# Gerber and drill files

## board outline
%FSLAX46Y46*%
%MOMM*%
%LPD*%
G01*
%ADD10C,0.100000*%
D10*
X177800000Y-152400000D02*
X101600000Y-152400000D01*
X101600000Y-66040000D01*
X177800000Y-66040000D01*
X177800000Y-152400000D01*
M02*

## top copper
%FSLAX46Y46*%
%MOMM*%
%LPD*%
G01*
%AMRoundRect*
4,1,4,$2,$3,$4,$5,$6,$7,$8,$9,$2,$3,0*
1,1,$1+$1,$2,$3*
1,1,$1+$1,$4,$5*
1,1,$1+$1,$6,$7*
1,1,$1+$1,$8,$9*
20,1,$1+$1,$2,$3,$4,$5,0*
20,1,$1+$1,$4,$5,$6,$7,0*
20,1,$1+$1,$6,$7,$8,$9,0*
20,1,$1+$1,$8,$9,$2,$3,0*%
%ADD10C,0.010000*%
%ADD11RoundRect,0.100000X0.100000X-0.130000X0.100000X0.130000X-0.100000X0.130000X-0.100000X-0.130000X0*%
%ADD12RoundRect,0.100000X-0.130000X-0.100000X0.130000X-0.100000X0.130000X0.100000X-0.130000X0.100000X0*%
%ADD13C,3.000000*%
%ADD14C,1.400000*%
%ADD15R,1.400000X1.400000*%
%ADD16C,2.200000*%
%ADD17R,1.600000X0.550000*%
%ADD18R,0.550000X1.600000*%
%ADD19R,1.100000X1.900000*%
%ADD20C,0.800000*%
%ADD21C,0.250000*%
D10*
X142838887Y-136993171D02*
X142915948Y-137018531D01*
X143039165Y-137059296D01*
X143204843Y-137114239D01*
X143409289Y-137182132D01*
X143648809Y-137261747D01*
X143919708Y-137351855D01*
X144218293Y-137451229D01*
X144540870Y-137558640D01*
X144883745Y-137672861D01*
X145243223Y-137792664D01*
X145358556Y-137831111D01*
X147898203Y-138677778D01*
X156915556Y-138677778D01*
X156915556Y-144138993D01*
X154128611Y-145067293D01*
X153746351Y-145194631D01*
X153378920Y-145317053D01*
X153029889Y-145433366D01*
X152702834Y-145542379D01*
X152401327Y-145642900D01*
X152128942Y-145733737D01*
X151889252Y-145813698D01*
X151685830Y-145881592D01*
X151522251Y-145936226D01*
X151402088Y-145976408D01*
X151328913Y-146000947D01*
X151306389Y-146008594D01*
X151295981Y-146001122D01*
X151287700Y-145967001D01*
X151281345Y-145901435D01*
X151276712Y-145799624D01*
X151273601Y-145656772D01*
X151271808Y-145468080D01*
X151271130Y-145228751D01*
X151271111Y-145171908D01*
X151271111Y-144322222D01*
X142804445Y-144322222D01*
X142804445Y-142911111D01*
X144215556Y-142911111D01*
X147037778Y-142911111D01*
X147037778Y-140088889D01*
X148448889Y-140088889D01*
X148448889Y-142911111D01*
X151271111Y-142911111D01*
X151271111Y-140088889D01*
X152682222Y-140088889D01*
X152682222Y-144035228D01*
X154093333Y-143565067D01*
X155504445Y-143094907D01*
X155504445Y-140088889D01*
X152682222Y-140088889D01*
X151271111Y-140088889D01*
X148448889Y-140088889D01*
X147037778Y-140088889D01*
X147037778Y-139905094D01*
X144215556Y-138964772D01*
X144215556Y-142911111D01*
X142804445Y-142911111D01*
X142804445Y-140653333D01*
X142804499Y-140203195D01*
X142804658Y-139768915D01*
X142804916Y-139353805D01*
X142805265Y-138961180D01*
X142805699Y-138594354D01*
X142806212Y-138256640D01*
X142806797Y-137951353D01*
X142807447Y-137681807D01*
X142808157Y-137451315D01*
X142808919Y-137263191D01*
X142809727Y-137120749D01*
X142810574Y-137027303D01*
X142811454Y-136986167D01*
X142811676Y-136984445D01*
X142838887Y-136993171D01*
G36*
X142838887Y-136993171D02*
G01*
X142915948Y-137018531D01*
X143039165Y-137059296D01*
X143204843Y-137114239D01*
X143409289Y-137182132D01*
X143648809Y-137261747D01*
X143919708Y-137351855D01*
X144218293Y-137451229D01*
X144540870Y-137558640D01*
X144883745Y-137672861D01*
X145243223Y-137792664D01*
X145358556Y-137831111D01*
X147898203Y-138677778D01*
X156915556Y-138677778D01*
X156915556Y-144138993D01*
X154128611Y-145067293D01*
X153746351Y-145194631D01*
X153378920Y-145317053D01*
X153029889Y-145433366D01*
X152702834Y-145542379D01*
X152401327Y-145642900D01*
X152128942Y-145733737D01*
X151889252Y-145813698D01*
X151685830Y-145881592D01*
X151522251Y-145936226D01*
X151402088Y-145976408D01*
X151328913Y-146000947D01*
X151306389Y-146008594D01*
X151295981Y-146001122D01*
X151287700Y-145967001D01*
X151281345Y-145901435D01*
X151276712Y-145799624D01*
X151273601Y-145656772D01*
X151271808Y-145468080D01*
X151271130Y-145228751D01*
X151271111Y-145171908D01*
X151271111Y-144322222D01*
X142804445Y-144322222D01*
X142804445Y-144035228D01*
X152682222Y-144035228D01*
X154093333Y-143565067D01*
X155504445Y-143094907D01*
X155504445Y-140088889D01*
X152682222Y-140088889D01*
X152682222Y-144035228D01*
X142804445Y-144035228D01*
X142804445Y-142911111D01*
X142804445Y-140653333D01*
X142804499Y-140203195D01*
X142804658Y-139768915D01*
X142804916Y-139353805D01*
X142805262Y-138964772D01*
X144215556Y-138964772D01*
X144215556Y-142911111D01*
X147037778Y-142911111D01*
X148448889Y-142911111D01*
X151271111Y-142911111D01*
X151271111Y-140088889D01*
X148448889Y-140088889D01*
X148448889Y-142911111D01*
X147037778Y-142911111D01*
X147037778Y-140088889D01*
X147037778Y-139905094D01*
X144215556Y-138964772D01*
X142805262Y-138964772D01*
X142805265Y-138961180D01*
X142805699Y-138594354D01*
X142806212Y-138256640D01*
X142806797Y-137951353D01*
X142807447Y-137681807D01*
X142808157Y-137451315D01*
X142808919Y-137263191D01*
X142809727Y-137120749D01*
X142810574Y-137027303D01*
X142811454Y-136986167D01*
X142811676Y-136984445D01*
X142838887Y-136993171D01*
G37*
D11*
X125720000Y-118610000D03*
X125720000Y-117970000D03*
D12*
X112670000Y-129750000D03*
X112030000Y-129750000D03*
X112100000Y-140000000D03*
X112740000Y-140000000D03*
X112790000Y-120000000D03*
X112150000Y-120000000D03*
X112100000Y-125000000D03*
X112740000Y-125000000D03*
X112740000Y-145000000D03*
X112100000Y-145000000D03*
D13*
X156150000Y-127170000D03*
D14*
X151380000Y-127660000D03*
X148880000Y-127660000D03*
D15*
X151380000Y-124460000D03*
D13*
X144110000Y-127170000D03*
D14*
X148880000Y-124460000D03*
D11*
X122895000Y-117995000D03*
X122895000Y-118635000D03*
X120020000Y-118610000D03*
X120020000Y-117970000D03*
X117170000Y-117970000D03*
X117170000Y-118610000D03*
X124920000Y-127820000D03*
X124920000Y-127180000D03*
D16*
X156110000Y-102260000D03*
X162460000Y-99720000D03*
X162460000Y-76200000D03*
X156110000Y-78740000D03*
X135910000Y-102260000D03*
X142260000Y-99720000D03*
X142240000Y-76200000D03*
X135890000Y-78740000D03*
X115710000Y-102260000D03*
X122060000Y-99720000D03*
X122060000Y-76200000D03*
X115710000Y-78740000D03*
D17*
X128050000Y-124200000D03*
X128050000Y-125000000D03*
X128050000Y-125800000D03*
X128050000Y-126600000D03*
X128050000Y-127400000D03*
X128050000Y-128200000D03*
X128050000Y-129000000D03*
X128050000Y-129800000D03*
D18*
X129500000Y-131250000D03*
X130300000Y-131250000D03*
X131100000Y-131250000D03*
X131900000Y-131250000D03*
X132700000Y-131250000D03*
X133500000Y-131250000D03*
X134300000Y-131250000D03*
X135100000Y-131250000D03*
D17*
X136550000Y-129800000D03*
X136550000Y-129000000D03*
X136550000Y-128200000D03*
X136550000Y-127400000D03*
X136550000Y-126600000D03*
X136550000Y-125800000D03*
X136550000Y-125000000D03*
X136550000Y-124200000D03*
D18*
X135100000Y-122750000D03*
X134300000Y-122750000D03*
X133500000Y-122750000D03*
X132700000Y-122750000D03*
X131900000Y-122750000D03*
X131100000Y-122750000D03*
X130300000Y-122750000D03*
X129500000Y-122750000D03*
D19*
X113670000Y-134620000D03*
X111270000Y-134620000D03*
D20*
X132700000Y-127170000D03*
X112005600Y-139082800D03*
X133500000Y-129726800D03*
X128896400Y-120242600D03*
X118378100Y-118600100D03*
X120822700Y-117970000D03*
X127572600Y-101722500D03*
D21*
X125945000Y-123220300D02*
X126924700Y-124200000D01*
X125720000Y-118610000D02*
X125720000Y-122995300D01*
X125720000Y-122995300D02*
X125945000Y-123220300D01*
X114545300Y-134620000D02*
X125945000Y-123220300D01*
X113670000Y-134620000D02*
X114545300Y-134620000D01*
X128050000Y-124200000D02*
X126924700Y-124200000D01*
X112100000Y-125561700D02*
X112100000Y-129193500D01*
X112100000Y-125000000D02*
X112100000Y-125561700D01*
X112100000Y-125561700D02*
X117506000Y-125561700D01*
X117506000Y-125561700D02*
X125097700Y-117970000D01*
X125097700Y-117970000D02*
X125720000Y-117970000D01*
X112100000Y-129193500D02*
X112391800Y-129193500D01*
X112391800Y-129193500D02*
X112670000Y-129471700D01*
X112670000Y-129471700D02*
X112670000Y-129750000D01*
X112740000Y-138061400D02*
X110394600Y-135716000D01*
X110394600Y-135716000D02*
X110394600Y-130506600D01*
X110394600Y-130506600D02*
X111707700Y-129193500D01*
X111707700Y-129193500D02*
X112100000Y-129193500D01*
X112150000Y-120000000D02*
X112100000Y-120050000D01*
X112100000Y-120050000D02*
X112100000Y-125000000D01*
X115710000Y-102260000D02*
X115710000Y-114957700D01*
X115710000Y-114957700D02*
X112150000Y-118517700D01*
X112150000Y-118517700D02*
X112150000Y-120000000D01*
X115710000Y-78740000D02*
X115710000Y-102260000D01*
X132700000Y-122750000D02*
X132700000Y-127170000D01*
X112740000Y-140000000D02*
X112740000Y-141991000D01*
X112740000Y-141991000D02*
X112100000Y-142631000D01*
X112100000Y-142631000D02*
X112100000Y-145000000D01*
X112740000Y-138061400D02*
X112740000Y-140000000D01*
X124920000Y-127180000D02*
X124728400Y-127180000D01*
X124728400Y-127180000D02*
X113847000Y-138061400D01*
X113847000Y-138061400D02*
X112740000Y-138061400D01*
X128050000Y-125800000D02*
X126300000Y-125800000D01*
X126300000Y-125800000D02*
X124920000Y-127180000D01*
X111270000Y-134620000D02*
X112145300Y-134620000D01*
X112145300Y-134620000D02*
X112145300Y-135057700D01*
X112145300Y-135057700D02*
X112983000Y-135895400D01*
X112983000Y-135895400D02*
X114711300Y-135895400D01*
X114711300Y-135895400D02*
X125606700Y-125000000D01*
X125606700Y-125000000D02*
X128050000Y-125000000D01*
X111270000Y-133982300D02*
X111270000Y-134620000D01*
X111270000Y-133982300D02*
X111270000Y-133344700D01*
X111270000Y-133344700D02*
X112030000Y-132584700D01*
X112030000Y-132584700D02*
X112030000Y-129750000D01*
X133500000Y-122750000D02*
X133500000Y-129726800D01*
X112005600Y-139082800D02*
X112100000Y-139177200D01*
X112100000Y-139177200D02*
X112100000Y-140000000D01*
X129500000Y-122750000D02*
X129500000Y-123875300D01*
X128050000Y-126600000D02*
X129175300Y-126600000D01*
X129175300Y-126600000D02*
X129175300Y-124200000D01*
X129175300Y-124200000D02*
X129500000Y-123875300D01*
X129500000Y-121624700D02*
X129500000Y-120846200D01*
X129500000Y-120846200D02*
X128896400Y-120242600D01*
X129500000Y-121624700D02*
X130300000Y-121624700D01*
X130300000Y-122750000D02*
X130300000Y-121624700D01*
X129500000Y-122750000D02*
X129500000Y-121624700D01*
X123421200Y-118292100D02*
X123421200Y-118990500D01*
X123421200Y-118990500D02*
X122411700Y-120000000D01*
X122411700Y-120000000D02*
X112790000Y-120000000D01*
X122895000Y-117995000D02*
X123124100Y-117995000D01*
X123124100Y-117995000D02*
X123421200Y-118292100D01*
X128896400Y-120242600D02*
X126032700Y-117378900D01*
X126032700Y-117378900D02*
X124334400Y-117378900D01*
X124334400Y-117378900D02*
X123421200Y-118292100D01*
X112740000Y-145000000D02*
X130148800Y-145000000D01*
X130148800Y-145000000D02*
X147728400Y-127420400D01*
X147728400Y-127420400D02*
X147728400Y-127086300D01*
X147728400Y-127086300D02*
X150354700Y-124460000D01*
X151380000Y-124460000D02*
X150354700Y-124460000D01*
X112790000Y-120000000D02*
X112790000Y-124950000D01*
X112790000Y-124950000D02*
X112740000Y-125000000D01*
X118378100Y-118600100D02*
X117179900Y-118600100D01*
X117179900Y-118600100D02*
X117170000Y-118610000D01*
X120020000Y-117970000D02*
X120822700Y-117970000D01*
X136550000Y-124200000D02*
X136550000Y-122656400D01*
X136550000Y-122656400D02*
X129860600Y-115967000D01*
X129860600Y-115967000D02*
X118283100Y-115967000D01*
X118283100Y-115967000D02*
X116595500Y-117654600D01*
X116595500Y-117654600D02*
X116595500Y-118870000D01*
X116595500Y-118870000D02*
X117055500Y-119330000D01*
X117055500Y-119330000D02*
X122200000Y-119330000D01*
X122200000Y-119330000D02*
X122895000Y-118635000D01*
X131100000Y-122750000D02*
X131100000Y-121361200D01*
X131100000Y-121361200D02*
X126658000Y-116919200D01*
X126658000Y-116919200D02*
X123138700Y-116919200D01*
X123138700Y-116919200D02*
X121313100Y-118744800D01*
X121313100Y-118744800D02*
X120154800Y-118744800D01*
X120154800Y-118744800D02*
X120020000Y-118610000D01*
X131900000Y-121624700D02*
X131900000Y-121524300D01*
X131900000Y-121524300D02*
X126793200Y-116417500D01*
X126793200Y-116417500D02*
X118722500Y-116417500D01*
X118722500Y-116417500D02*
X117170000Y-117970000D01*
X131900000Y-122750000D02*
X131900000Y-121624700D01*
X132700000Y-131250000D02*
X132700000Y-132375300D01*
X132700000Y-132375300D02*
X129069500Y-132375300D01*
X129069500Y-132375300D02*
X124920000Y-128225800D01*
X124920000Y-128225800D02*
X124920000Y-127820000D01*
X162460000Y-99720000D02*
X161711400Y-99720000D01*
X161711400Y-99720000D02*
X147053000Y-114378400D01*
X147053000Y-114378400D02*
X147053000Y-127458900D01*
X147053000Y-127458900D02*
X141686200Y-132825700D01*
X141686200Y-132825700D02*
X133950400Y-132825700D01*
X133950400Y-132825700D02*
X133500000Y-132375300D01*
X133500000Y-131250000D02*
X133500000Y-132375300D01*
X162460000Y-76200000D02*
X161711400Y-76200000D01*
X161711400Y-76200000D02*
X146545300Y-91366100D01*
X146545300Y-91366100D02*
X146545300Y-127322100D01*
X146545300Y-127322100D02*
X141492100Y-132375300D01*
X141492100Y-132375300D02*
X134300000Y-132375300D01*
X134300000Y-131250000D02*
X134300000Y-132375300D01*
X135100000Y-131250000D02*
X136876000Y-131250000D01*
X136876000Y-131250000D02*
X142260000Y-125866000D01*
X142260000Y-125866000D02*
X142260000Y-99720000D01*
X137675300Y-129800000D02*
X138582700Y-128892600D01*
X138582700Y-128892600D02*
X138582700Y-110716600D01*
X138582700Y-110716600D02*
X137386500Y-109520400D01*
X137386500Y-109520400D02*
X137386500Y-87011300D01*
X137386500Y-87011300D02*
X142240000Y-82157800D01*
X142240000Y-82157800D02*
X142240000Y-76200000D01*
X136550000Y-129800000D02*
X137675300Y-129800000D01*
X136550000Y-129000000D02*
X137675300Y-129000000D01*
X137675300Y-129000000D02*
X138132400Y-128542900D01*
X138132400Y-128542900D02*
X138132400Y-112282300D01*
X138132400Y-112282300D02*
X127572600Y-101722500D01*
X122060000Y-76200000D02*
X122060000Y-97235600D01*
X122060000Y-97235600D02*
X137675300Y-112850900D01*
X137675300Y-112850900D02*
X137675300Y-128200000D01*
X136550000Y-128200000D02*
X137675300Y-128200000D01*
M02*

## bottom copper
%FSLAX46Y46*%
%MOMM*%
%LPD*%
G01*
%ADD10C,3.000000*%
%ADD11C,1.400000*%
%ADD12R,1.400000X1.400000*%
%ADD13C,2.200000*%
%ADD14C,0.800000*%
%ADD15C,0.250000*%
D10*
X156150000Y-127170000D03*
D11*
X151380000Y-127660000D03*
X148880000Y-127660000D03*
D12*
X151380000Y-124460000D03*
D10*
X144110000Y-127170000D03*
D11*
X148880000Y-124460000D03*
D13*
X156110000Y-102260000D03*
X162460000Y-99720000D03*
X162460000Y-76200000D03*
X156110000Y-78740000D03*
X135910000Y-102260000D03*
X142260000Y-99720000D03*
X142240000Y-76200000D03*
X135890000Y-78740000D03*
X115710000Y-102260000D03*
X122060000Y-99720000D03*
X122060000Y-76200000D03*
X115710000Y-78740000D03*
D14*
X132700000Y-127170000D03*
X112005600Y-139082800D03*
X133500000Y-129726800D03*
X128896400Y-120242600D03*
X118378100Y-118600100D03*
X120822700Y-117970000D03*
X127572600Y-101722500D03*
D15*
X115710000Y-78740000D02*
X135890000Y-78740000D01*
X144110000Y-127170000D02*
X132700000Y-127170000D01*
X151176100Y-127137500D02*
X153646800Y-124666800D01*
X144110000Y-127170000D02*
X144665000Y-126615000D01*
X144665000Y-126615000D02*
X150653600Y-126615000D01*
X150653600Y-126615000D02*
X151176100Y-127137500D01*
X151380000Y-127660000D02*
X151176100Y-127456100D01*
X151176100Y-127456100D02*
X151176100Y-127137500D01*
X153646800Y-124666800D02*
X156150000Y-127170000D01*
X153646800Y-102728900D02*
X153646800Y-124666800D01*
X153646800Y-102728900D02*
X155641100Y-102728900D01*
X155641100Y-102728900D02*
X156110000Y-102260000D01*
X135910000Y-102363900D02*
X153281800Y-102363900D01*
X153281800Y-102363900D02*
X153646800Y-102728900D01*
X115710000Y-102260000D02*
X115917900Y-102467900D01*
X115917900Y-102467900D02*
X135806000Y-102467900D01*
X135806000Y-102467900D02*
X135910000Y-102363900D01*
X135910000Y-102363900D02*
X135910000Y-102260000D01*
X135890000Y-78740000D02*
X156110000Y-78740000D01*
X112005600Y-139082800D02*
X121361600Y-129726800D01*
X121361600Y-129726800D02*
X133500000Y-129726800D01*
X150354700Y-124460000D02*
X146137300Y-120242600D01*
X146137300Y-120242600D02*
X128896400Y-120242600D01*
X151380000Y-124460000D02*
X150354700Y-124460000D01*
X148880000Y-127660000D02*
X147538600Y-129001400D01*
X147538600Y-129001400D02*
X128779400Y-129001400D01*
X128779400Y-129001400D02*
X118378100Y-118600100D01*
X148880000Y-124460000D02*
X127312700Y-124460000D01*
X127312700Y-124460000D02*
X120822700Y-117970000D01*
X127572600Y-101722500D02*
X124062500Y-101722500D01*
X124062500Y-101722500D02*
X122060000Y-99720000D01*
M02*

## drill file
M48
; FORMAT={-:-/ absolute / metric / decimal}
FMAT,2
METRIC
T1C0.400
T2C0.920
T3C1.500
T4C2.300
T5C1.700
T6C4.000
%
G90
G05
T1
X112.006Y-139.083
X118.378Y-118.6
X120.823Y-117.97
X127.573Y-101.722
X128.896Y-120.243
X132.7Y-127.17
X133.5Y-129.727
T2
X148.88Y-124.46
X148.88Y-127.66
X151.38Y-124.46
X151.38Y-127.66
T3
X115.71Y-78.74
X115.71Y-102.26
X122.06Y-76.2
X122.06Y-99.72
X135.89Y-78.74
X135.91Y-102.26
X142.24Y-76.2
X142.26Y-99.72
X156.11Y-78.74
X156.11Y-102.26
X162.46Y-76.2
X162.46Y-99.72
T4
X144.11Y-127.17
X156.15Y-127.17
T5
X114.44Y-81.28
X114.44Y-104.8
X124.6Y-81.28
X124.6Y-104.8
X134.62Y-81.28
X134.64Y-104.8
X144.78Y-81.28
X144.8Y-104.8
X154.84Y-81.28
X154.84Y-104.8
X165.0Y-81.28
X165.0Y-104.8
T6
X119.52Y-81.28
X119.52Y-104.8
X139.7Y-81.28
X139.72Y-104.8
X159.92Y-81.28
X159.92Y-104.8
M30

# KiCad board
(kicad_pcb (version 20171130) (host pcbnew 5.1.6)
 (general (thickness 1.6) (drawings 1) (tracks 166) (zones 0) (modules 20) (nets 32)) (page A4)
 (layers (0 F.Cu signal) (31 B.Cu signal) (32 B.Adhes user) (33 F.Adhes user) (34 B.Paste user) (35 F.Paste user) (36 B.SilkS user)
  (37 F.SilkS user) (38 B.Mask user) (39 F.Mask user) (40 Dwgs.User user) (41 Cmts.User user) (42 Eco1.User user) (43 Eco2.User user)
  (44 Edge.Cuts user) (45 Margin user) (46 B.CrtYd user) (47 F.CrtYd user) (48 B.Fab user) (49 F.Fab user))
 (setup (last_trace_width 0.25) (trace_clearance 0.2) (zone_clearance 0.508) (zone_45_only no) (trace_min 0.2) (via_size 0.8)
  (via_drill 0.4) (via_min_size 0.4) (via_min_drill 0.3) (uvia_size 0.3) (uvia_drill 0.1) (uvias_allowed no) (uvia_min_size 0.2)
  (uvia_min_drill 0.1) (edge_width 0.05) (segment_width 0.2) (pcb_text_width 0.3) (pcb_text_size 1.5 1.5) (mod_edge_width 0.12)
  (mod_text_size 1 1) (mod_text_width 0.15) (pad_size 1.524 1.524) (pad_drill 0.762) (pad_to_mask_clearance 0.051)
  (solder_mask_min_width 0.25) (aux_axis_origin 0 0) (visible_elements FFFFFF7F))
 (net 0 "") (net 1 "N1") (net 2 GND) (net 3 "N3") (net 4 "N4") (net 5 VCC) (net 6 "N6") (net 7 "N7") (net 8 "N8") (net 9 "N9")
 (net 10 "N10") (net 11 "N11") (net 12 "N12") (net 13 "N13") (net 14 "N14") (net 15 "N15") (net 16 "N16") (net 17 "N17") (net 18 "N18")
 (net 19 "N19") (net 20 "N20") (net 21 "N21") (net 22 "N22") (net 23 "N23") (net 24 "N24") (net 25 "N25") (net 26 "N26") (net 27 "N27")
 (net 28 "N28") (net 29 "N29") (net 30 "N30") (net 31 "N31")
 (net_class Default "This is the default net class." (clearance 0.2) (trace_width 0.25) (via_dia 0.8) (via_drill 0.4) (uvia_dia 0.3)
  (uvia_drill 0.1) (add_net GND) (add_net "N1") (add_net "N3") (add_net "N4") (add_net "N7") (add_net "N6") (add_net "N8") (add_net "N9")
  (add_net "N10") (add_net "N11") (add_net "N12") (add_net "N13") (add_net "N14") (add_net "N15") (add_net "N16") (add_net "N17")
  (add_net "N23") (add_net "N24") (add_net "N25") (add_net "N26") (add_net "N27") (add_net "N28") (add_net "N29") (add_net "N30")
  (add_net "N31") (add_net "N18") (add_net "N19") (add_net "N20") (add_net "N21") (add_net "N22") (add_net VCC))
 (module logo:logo (layer F.Cu) (at 149.86 141.5)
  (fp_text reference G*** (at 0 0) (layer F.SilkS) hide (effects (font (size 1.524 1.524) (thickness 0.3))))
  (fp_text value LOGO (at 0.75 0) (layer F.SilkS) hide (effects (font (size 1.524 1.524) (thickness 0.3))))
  (fp_poly
   (pts (xy -7.021113 -4.506829) (xy -6.944052 -4.481469) (xy -6.820835 -4.440704) (xy -6.655157 -4.385761) (xy -6.450711 -4.317868)
    (xy -6.211191 -4.238253) (xy -5.940292 -4.148145) (xy -5.641707 -4.048771) (xy -5.31913 -3.94136) (xy -4.976255 -3.827139)
    (xy -4.616777 -3.707336) (xy -4.501444 -3.668889) (xy -1.961797 -2.822222) (xy 7.055556 -2.822222) (xy 7.055556 2.638993)
    (xy 4.268611 3.567293) (xy 3.886351 3.694631) (xy 3.51892 3.817053) (xy 3.169889 3.933366) (xy 2.842834 4.042379) (xy 2.541327 4.1429)
    (xy 2.268942 4.233737) (xy 2.029252 4.313698) (xy 1.82583 4.381592) (xy 1.662251 4.436226) (xy 1.542088 4.476408) (xy 1.468913 4.500947)
    (xy 1.446389 4.508594) (xy 1.435981 4.501122) (xy 1.4277 4.467001) (xy 1.421345 4.401435) (xy 1.416712 4.299624) (xy 1.413601 4.156772)
    (xy 1.411808 3.96808) (xy 1.41113 3.728751) (xy 1.411111 3.671908) (xy 1.411111 2.822222) (xy -7.055555 2.822222)
    (xy -7.055555 1.411111) (xy -5.644444 1.411111) (xy -2.822222 1.411111) (xy -2.822222 -1.411111) (xy -1.411111 -1.411111)
    (xy -1.411111 1.411111) (xy 1.411111 1.411111) (xy 1.411111 -1.411111) (xy 2.822222 -1.411111) (xy 2.822222 2.535228)
    (xy 4.233333 2.065067) (xy 5.644445 1.594907) (xy 5.644445 -1.411111) (xy 2.822222 -1.411111) (xy 1.411111 -1.411111)
    (xy -1.411111 -1.411111) (xy -2.822222 -1.411111) (xy -2.822222 -1.594906) (xy -5.644444 -2.535228) (xy -5.644444 1.411111)
    (xy -7.055555 1.411111) (xy -7.055555 -0.846667) (xy -7.055501 -1.296805) (xy -7.055342 -1.731085) (xy -7.055084 -2.146195)
    (xy -7.054735 -2.53882) (xy -7.054301 -2.905646) (xy -7.053788 -3.24336) (xy -7.053203 -3.548647) (xy -7.052553 -3.818193)
    (xy -7.051843 -4.048685) (xy -7.051081 -4.236809) (xy -7.050273 -4.379251) (xy -7.049426 -4.472697) (xy -7.048546 -4.513833)
    (xy -7.048324 -4.515555) (xy -7.021113 -4.506829))
   (layer F.Cu) (width 0.01)))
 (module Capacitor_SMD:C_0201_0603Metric (layer F.Cu) (at 125.72 118.29 90)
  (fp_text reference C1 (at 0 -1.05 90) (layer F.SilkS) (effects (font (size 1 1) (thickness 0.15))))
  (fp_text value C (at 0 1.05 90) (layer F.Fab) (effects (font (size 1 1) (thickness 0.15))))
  (pad "" smd roundrect (at -0.345 0 90) (size 0.318 0.36) (layers F.Paste) (roundrect_rratio 0.25))
  (pad "" smd roundrect (at 0.345 0 90) (size 0.318 0.36) (layers F.Paste) (roundrect_rratio 0.25))
  (pad 1 smd roundrect (at -0.32 0 90) (size 0.46 0.4) (layers F.Cu F.Mask) (roundrect_rratio 0.25) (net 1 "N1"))
  (pad 2 smd roundrect (at 0.32 0 90) (size 0.46 0.4) (layers F.Cu F.Mask) (roundrect_rratio 0.25) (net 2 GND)))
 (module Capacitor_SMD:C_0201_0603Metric (layer F.Cu) (at 112.35 129.75)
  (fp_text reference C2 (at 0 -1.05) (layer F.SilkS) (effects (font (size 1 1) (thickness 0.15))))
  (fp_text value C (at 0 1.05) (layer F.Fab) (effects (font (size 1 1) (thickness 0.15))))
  (pad 2 smd roundrect (at 0.32 0) (size 0.46 0.4) (layers F.Cu F.Mask) (roundrect_rratio 0.25) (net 2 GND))
  (pad 1 smd roundrect (at -0.32 0) (size 0.46 0.4) (layers F.Cu F.Mask) (roundrect_rratio 0.25) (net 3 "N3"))
  (pad "" smd roundrect (at 0.345 0) (size 0.318 0.36) (layers F.Paste) (roundrect_rratio 0.25))
  (pad "" smd roundrect (at -0.345 0) (size 0.318 0.36) (layers F.Paste) (roundrect_rratio 0.25)))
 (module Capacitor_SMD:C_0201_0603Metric (layer F.Cu) (at 112.42 140)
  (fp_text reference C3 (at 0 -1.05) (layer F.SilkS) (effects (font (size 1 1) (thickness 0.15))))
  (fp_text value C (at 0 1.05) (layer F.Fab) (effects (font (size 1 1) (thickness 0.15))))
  (pad "" smd roundrect (at -0.345 0) (size 0.318 0.36) (layers F.Paste) (roundrect_rratio 0.25))
  (pad "" smd roundrect (at 0.345 0) (size 0.318 0.36) (layers F.Paste) (roundrect_rratio 0.25))
  (pad 1 smd roundrect (at -0.32 0) (size 0.46 0.4) (layers F.Cu F.Mask) (roundrect_rratio 0.25) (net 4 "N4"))
  (pad 2 smd roundrect (at 0.32 0) (size 0.46 0.4) (layers F.Cu F.Mask) (roundrect_rratio 0.25) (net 2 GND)))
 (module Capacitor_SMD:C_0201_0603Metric (layer F.Cu) (at 112.47 120)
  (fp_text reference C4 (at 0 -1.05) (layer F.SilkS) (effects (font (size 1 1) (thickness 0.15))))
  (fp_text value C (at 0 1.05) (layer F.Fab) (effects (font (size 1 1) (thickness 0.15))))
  (pad 2 smd roundrect (at 0.32 0) (size 0.46 0.4) (layers F.Cu F.Mask) (roundrect_rratio 0.25) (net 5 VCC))
  (pad 1 smd roundrect (at -0.32 0) (size 0.46 0.4) (layers F.Cu F.Mask) (roundrect_rratio 0.25) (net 2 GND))
  (pad "" smd roundrect (at 0.345 0) (size 0.318 0.36) (layers F.Paste) (roundrect_rratio 0.25))
  (pad "" smd roundrect (at -0.345 0) (size 0.318 0.36) (layers F.Paste) (roundrect_rratio 0.25)))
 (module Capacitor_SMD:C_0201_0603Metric (layer F.Cu) (at 112.42 125)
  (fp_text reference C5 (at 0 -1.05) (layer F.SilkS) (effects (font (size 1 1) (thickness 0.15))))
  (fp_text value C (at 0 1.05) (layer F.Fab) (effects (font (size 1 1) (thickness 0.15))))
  (pad "" smd roundrect (at -0.345 0) (size 0.318 0.36) (layers F.Paste) (roundrect_rratio 0.25))
  (pad "" smd roundrect (at 0.345 0) (size 0.318 0.36) (layers F.Paste) (roundrect_rratio 0.25))
  (pad 1 smd roundrect (at -0.32 0) (size 0.46 0.4) (layers F.Cu F.Mask) (roundrect_rratio 0.25) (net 2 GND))
  (pad 2 smd roundrect (at 0.32 0) (size 0.46 0.4) (layers F.Cu F.Mask) (roundrect_rratio 0.25) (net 5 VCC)))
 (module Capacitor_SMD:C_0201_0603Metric (layer F.Cu) (at 112.42 145)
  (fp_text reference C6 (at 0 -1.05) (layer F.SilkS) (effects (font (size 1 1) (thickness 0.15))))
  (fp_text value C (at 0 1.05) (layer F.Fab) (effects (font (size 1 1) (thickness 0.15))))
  (pad 2 smd roundrect (at 0.32 0) (size 0.46 0.4) (layers F.Cu F.Mask) (roundrect_rratio 0.25) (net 5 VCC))
  (pad 1 smd roundrect (at -0.32 0) (size 0.46 0.4) (layers F.Cu F.Mask) (roundrect_rratio 0.25) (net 2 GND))
  (pad "" smd roundrect (at 0.345 0) (size 0.318 0.36) (layers F.Paste) (roundrect_rratio 0.25))
  (pad "" smd roundrect (at -0.345 0) (size 0.318 0.36) (layers F.Paste) (roundrect_rratio 0.25)))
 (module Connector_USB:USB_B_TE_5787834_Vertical (layer F.Cu) (at 151.38 124.46)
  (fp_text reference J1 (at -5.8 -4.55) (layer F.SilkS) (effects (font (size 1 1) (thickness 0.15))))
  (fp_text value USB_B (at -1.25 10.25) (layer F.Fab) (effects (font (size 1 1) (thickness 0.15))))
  (pad 5 thru_hole circle (at 4.77 2.71) (size 3 3) (drill 2.3) (layers *.Cu *.Mask) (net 2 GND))
  (pad 4 thru_hole circle (at 0 3.2) (size 1.4 1.4) (drill 0.92) (layers *.Cu *.Mask) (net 2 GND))
  (pad 3 thru_hole circle (at -2.5 3.2) (size 1.4 1.4) (drill 0.92) (layers *.Cu *.Mask) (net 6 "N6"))
  (pad 1 thru_hole rect (at 0 0) (size 1.4 1.4) (drill 0.92) (layers *.Cu *.Mask) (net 5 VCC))
  (pad 5 thru_hole circle (at -7.27 2.71) (size 3 3) (drill 2.3) (layers *.Cu *.Mask) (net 2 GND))
  (pad 2 thru_hole circle (at -2.5 0) (size 1.4 1.4) (drill 0.92) (layers *.Cu *.Mask) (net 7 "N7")))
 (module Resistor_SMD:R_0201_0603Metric (layer F.Cu) (at 122.895 118.315 90)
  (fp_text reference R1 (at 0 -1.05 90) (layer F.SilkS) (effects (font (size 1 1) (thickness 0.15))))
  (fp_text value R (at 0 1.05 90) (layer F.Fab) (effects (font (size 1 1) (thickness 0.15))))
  (pad 2 smd roundrect (at 0.32 0 90) (size 0.46 0.4) (layers F.Cu F.Mask) (roundrect_rratio 0.25) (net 5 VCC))
  (pad 1 smd roundrect (at -0.32 0 90) (size 0.46 0.4) (layers F.Cu F.Mask) (roundrect_rratio 0.25) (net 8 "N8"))
  (pad "" smd roundrect (at 0.345 0 90) (size 0.318 0.36) (layers F.Paste) (roundrect_rratio 0.25))
  (pad "" smd roundrect (at -0.345 0 90) (size 0.318 0.36) (layers F.Paste) (roundrect_rratio 0.25)))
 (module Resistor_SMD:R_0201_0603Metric (layer F.Cu) (at 120.02 118.29 90)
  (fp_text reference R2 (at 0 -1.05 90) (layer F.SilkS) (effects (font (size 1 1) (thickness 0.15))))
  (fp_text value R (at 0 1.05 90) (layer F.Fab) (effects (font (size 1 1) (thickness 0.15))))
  (pad "" smd roundrect (at -0.345 0 90) (size 0.318 0.36) (layers F.Paste) (roundrect_rratio 0.25))
  (pad "" smd roundrect (at 0.345 0 90) (size 0.318 0.36) (layers F.Paste) (roundrect_rratio 0.25))
  (pad 1 smd roundrect (at -0.32 0 90) (size 0.46 0.4) (layers F.Cu F.Mask) (roundrect_rratio 0.25) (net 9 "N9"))
  (pad 2 smd roundrect (at 0.32 0 90) (size 0.46 0.4) (layers F.Cu F.Mask) (roundrect_rratio 0.25) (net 7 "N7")))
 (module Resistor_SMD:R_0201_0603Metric (layer F.Cu) (at 117.17 118.29 90)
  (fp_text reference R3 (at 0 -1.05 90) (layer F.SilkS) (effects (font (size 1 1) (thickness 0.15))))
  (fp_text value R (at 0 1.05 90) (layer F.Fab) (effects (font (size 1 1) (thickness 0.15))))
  (pad 2 smd roundrect (at 0.32 0 90) (size 0.46 0.4) (layers F.Cu F.Mask) (roundrect_rratio 0.25) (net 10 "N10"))
  (pad 1 smd roundrect (at -0.32 0 90) (size 0.46 0.4) (layers F.Cu F.Mask) (roundrect_rratio 0.25) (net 6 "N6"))
  (pad "" smd roundrect (at 0.345 0 90) (size 0.318 0.36) (layers F.Paste) (roundrect_rratio 0.25))
  (pad "" smd roundrect (at -0.345 0 90) (size 0.318 0.36) (layers F.Paste) (roundrect_rratio 0.25)))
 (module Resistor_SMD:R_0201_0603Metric (layer F.Cu) (at 124.92 127.5 90)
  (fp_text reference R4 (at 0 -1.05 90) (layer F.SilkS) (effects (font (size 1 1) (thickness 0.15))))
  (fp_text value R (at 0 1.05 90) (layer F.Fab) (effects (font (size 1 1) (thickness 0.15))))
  (pad "" smd roundrect (at -0.345 0 90) (size 0.318 0.36) (layers F.Paste) (roundrect_rratio 0.25))
  (pad "" smd roundrect (at 0.345 0 90) (size 0.318 0.36) (layers F.Paste) (roundrect_rratio 0.25))
  (pad 1 smd roundrect (at -0.32 0 90) (size 0.46 0.4) (layers F.Cu F.Mask) (roundrect_rratio 0.25) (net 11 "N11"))
  (pad 2 smd roundrect (at 0.32 0 90) (size 0.46 0.4) (layers F.Cu F.Mask) (roundrect_rratio 0.25) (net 2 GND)))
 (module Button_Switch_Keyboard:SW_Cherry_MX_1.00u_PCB (layer F.Cu) (at 162.46 99.72)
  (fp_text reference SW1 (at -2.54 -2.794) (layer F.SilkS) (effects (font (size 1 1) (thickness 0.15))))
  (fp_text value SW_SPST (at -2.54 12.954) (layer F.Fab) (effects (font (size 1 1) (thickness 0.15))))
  (pad "" np_thru_hole circle (at 2.54 5.08) (size 1.7 1.7) (drill 1.7) (layers *.Cu *.Mask))
  (pad "" np_thru_hole circle (at -7.62 5.08) (size 1.7 1.7) (drill 1.7) (layers *.Cu *.Mask))
  (pad "" np_thru_hole circle (at -2.54 5.08) (size 4 4) (drill 4) (layers *.Cu *.Mask))
  (pad 2 thru_hole circle (at -6.35 2.54) (size 2.2 2.2) (drill 1.5) (layers *.Cu *.Mask) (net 2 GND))
  (pad 1 thru_hole circle (at 0 0) (size 2.2 2.2) (drill 1.5) (layers *.Cu *.Mask) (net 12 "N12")))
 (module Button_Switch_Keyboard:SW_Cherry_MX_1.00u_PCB (layer F.Cu) (at 162.46 76.2)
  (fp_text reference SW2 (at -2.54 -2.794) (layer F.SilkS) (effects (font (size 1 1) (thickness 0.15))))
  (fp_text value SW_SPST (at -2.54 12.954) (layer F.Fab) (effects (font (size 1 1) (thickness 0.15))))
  (pad 1 thru_hole circle (at 0 0) (size 2.2 2.2) (drill 1.5) (layers *.Cu *.Mask) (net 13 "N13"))
  (pad 2 thru_hole circle (at -6.35 2.54) (size 2.2 2.2) (drill 1.5) (layers *.Cu *.Mask) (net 2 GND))
  (pad "" np_thru_hole circle (at -2.54 5.08) (size 4 4) (drill 4) (layers *.Cu *.Mask))
  (pad "" np_thru_hole circle (at -7.62 5.08) (size 1.7 1.7) (drill 1.7) (layers *.Cu *.Mask))
  (pad "" np_thru_hole circle (at 2.54 5.08) (size 1.7 1.7) (drill 1.7) (layers *.Cu *.Mask)))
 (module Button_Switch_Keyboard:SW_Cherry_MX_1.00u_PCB (layer F.Cu) (at 142.26 99.72)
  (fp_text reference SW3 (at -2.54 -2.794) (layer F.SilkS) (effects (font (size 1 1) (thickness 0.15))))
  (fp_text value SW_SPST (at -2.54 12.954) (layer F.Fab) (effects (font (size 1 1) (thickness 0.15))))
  (pad "" np_thru_hole circle (at 2.54 5.08) (size 1.7 1.7) (drill 1.7) (layers *.Cu *.Mask))
  (pad "" np_thru_hole circle (at -7.62 5.08) (size 1.7 1.7) (drill 1.7) (layers *.Cu *.Mask))
  (pad "" np_thru_hole circle (at -2.54 5.08) (size 4 4) (drill 4) (layers *.Cu *.Mask))
  (pad 2 thru_hole circle (at -6.35 2.54) (size 2.2 2.2) (drill 1.5) (layers *.Cu *.Mask) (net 2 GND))
  (pad 1 thru_hole circle (at 0 0) (size 2.2 2.2) (drill 1.5) (layers *.Cu *.Mask) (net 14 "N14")))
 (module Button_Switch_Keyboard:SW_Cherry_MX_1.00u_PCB (layer F.Cu) (at 142.24 76.2)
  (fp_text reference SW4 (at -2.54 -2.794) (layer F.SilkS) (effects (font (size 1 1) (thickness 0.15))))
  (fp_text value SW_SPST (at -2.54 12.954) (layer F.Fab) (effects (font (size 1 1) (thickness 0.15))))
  (pad 1 thru_hole circle (at 0 0) (size 2.2 2.2) (drill 1.5) (layers *.Cu *.Mask) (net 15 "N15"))
  (pad 2 thru_hole circle (at -6.35 2.54) (size 2.2 2.2) (drill 1.5) (layers *.Cu *.Mask) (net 2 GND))
  (pad "" np_thru_hole circle (at -2.54 5.08) (size 4 4) (drill 4) (layers *.Cu *.Mask))
  (pad "" np_thru_hole circle (at -7.62 5.08) (size 1.7 1.7) (drill 1.7) (layers *.Cu *.Mask))
  (pad "" np_thru_hole circle (at 2.54 5.08) (size 1.7 1.7) (drill 1.7) (layers *.Cu *.Mask)))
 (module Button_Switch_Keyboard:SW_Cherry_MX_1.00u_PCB (layer F.Cu) (at 122.06 99.72)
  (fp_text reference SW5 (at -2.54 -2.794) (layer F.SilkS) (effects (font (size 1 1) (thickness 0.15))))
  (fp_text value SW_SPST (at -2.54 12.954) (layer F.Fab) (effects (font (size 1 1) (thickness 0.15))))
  (pad "" np_thru_hole circle (at 2.54 5.08) (size 1.7 1.7) (drill 1.7) (layers *.Cu *.Mask))
  (pad "" np_thru_hole circle (at -7.62 5.08) (size 1.7 1.7) (drill 1.7) (layers *.Cu *.Mask))
  (pad "" np_thru_hole circle (at -2.54 5.08) (size 4 4) (drill 4) (layers *.Cu *.Mask))
  (pad 2 thru_hole circle (at -6.35 2.54) (size 2.2 2.2) (drill 1.5) (layers *.Cu *.Mask) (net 2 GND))
  (pad 1 thru_hole circle (at 0 0) (size 2.2 2.2) (drill 1.5) (layers *.Cu *.Mask) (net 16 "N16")))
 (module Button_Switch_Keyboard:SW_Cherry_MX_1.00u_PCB (layer F.Cu) (at 122.06 76.2)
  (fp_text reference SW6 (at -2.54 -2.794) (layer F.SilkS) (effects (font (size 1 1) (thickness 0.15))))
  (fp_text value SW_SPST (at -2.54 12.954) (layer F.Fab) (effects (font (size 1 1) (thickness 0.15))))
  (pad 1 thru_hole circle (at 0 0) (size 2.2 2.2) (drill 1.5) (layers *.Cu *.Mask) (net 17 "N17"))
  (pad 2 thru_hole circle (at -6.35 2.54) (size 2.2 2.2) (drill 1.5) (layers *.Cu *.Mask) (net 2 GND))
  (pad "" np_thru_hole circle (at -2.54 5.08) (size 4 4) (drill 4) (layers *.Cu *.Mask))
  (pad "" np_thru_hole circle (at -7.62 5.08) (size 1.7 1.7) (drill 1.7) (layers *.Cu *.Mask))
  (pad "" np_thru_hole circle (at 2.54 5.08) (size 1.7 1.7) (drill 1.7) (layers *.Cu *.Mask)))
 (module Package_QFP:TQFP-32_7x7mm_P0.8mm (layer F.Cu) (at 132.3 127)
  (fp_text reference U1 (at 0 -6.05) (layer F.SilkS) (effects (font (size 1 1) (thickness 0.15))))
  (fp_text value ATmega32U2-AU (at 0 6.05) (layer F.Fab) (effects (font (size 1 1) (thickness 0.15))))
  (pad 1 smd rect (at -4.25 -2.8) (size 1.6 0.55) (layers F.Cu F.Paste F.Mask) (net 1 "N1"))
  (pad 2 smd rect (at -4.25 -2) (size 1.6 0.55) (layers F.Cu F.Paste F.Mask) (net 3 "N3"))
  (pad 3 smd rect (at -4.25 -1.2) (size 1.6 0.55) (layers F.Cu F.Paste F.Mask) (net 2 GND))
  (pad 4 smd rect (at -4.25 -0.4) (size 1.6 0.55) (layers F.Cu F.Paste F.Mask) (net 5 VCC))
  (pad 5 smd rect (at -4.25 0.4) (size 1.6 0.55) (layers F.Cu F.Paste F.Mask) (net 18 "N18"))
  (pad 6 smd rect (at -4.25 1.2) (size 1.6 0.55) (layers F.Cu F.Paste F.Mask) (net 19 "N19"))
  (pad 7 smd rect (at -4.25 2) (size 1.6 0.55) (layers F.Cu F.Paste F.Mask) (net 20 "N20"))
  (pad 8 smd rect (at -4.25 2.8) (size 1.6 0.55) (layers F.Cu F.Paste F.Mask) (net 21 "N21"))
  (pad 9 smd rect (at -2.8 4.25 90) (size 1.6 0.55) (layers F.Cu F.Paste F.Mask) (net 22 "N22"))
  (pad 10 smd rect (at -2 4.25 90) (size 1.6 0.55) (layers F.Cu F.Paste F.Mask) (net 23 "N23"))
  (pad 11 smd rect (at -1.2 4.25 90) (size 1.6 0.55) (layers F.Cu F.Paste F.Mask) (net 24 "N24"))
  (pad 12 smd rect (at -0.4 4.25 90) (size 1.6 0.55) (layers F.Cu F.Paste F.Mask) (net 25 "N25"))
  (pad 13 smd rect (at 0.4 4.25 90) (size 1.6 0.55) (layers F.Cu F.Paste F.Mask) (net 11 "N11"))
  (pad 14 smd rect (at 1.2 4.25 90) (size 1.6 0.55) (layers F.Cu F.Paste F.Mask) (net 12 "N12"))
  (pad 15 smd rect (at 2 4.25 90) (size 1.6 0.55) (layers F.Cu F.Paste F.Mask) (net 13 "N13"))
  (pad 16 smd rect (at 2.8 4.25 90) (size 1.6 0.55) (layers F.Cu F.Paste F.Mask) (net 14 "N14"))
  (pad 17 smd rect (at 4.25 2.8) (size 1.6 0.55) (layers F.Cu F.Paste F.Mask) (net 15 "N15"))
  (pad 18 smd rect (at 4.25 2) (size 1.6 0.55) (layers F.Cu F.Paste F.Mask) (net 16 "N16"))
  (pad 19 smd rect (at 4.25 1.2) (size 1.6 0.55) (layers F.Cu F.Paste F.Mask) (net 17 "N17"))
  (pad 20 smd rect (at 4.25 0.4) (size 1.6 0.55) (layers F.Cu F.Paste F.Mask) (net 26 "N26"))
  (pad 21 smd rect (at 4.25 -0.4) (size 1.6 0.55) (layers F.Cu F.Paste F.Mask) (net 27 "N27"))
  (pad 22 smd rect (at 4.25 -1.2) (size 1.6 0.55) (layers F.Cu F.Paste F.Mask) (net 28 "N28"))
  (pad 23 smd rect (at 4.25 -2) (size 1.6 0.55) (layers F.Cu F.Paste F.Mask) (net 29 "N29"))
  (pad 24 smd rect (at 4.25 -2.8) (size 1.6 0.55) (layers F.Cu F.Paste F.Mask) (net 8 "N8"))
  (pad 25 smd rect (at 2.8 -4.25 90) (size 1.6 0.55) (layers F.Cu F.Paste F.Mask) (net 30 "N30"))
  (pad 26 smd rect (at 2 -4.25 90) (size 1.6 0.55) (layers F.Cu F.Paste F.Mask) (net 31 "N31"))
  (pad 27 smd rect (at 1.2 -4.25 90) (size 1.6 0.55) (layers F.Cu F.Paste F.Mask) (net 4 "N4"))
  (pad 28 smd rect (at 0.4 -4.25 90) (size 1.6 0.55) (layers F.Cu F.Paste F.Mask) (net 2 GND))
  (pad 29 smd rect (at -0.4 -4.25 90) (size 1.6 0.55) (layers F.Cu F.Paste F.Mask) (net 10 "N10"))
  (pad 30 smd rect (at -1.2 -4.25 90) (size 1.6 0.55) (layers F.Cu F.Paste F.Mask) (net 9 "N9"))
  (pad 31 smd rect (at -2 -4.25 90) (size 1.6 0.55) (layers F.Cu F.Paste F.Mask) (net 5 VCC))
  (pad 32 smd rect (at -2.8 -4.25 90) (size 1.6 0.55) (layers F.Cu F.Paste F.Mask) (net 5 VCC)))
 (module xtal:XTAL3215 (layer F.Cu) (at 112.47 134.62)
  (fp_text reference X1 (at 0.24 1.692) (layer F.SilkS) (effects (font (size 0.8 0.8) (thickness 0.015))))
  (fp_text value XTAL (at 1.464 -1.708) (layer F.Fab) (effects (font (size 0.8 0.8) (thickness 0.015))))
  (pad P$1 smd rect (at 1.2 0) (size 1.1 1.9) (layers F.Cu F.Paste F.Mask) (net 1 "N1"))
  (pad P$2 smd rect (at -1.2 0) (size 1.1 1.9) (layers F.Cu F.Paste F.Mask) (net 3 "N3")))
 (gr_poly (pts (xy 177.8 152.4) (xy 101.6 152.4) (xy 101.6 66.04) (xy 177.8 66.04)) (layer Edge.Cuts) (width 0.1))
 (segment (start 125.945 123.2203) (end 126.9247 124.2) (width 0.25) (layer F.Cu) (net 1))
 (segment (start 125.72 118.61) (end 125.72 122.9953) (width 0.25) (layer F.Cu) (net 1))
 (segment (start 125.72 122.9953) (end 125.945 123.2203) (width 0.25) (layer F.Cu) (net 1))
 (segment (start 114.5453 134.62) (end 125.945 123.2203) (width 0.25) (layer F.Cu) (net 1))
 (segment (start 113.67 134.62) (end 114.5453 134.62) (width 0.25) (layer F.Cu) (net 1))
 (segment (start 128.05 124.2) (end 126.9247 124.2) (width 0.25) (layer F.Cu) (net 1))
 (segment (start 112.1 125.5617) (end 112.1 129.1935) (width 0.25) (layer F.Cu) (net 2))
 (segment (start 112.1 125) (end 112.1 125.5617) (width 0.25) (layer F.Cu) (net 2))
 (segment (start 112.1 125.5617) (end 117.506 125.5617) (width 0.25) (layer F.Cu) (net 2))
 (segment (start 117.506 125.5617) (end 125.0977 117.97) (width 0.25) (layer F.Cu) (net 2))
 (segment (start 125.0977 117.97) (end 125.72 117.97) (width 0.25) (layer F.Cu) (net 2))
 (segment (start 112.1 129.1935) (end 112.3918 129.1935) (width 0.25) (layer F.Cu) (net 2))
 (segment (start 112.3918 129.1935) (end 112.67 129.4717) (width 0.25) (layer F.Cu) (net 2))
 (segment (start 112.67 129.4717) (end 112.67 129.75) (width 0.25) (layer F.Cu) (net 2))
 (segment (start 112.74 138.0614) (end 110.3946 135.716) (width 0.25) (layer F.Cu) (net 2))
 (segment (start 110.3946 135.716) (end 110.3946 130.5066) (width 0.25) (layer F.Cu) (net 2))
 (segment (start 110.3946 130.5066) (end 111.7077 129.1935) (width 0.25) (layer F.Cu) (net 2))
 (segment (start 111.7077 129.1935) (end 112.1 129.1935) (width 0.25) (layer F.Cu) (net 2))
 (segment (start 112.15 120) (end 112.1 120.05) (width 0.25) (layer F.Cu) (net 2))
 (segment (start 112.1 120.05) (end 112.1 125) (width 0.25) (layer F.Cu) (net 2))
 (segment (start 115.71 102.26) (end 115.71 114.9577) (width 0.25) (layer F.Cu) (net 2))
 (segment (start 115.71 114.9577) (end 112.15 118.5177) (width 0.25) (layer F.Cu) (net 2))
 (segment (start 112.15 118.5177) (end 112.15 120) (width 0.25) (layer F.Cu) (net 2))
 (segment (start 115.71 78.74) (end 115.71 102.26) (width 0.25) (layer F.Cu) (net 2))
 (segment (start 132.7 122.75) (end 132.7 127.17) (width 0.25) (layer F.Cu) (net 2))
 (segment (start 115.71 78.74) (end 135.89 78.74) (width 0.25) (layer B.Cu) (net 2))
 (segment (start 144.11 127.17) (end 132.7 127.17) (width 0.25) (layer B.Cu) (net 2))
 (segment (start 112.74 140) (end 112.74 141.991) (width 0.25) (layer F.Cu) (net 2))
 (segment (start 112.74 141.991) (end 112.1 142.631) (width 0.25) (layer F.Cu) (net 2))
 (segment (start 112.1 142.631) (end 112.1 145) (width 0.25) (layer F.Cu) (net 2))
 (segment (start 112.74 138.0614) (end 112.74 140) (width 0.25) (layer F.Cu) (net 2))
 (segment (start 151.1761 127.1375) (end 153.6468 124.6668) (width 0.25) (layer B.Cu) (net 2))
 (segment (start 144.11 127.17) (end 144.665 126.615) (width 0.25) (layer B.Cu) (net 2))
 (segment (start 144.665 126.615) (end 150.6536 126.615) (width 0.25) (layer B.Cu) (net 2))
 (segment (start 150.6536 126.615) (end 151.1761 127.1375) (width 0.25) (layer B.Cu) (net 2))
 (segment (start 151.38 127.66) (end 151.1761 127.4561) (width 0.25) (layer B.Cu) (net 2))
 (segment (start 151.1761 127.4561) (end 151.1761 127.1375) (width 0.25) (layer B.Cu) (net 2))
 (segment (start 153.6468 124.6668) (end 156.15 127.17) (width 0.25) (layer B.Cu) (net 2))
 (segment (start 153.6468 102.7289) (end 153.6468 124.6668) (width 0.25) (layer B.Cu) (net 2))
 (segment (start 153.6468 102.7289) (end 155.6411 102.7289) (width 0.25) (layer B.Cu) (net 2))
 (segment (start 155.6411 102.7289) (end 156.11 102.26) (width 0.25) (layer B.Cu) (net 2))
 (segment (start 135.91 102.3639) (end 153.2818 102.3639) (width 0.25) (layer B.Cu) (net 2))
 (segment (start 153.2818 102.3639) (end 153.6468 102.7289) (width 0.25) (layer B.Cu) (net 2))
 (segment (start 124.92 127.18) (end 124.7284 127.18) (width 0.25) (layer F.Cu) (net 2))
 (segment (start 124.7284 127.18) (end 113.847 138.0614) (width 0.25) (layer F.Cu) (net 2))
 (segment (start 113.847 138.0614) (end 112.74 138.0614) (width 0.25) (layer F.Cu) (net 2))
 (segment (start 128.05 125.8) (end 126.3 125.8) (width 0.25) (layer F.Cu) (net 2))
 (segment (start 126.3 125.8) (end 124.92 127.18) (width 0.25) (layer F.Cu) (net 2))
 (segment (start 115.71 102.26) (end 115.9179 102.4679) (width 0.25) (layer B.Cu) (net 2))
 (segment (start 115.9179 102.4679) (end 135.806 102.4679) (width 0.25) (layer B.Cu) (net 2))
 (segment (start 135.806 102.4679) (end 135.91 102.3639) (width 0.25) (layer B.Cu) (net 2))
 (segment (start 135.91 102.3639) (end 135.91 102.26) (width 0.25) (layer B.Cu) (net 2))
 (segment (start 135.89 78.74) (end 156.11 78.74) (width 0.25) (layer B.Cu) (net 2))
 (via (at 132.7 127.17) (size 0.8) (layers F.Cu B.Cu) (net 2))
 (segment (start 111.27 134.62) (end 112.1453 134.62) (width 0.25) (layer F.Cu) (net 3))
 (segment (start 112.1453 134.62) (end 112.1453 135.0577) (width 0.25) (layer F.Cu) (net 3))
 (segment (start 112.1453 135.0577) (end 112.983 135.8954) (width 0.25) (layer F.Cu) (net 3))
 (segment (start 112.983 135.8954) (end 114.7113 135.8954) (width 0.25) (layer F.Cu) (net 3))
 (segment (start 114.7113 135.8954) (end 125.6067 125) (width 0.25) (layer F.Cu) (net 3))
 (segment (start 125.6067 125) (end 128.05 125) (width 0.25) (layer F.Cu) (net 3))
 (segment (start 111.27 133.9823) (end 111.27 134.62) (width 0.25) (layer F.Cu) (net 3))
 (segment (start 111.27 133.9823) (end 111.27 133.3447) (width 0.25) (layer F.Cu) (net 3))
 (segment (start 111.27 133.3447) (end 112.03 132.5847) (width 0.25) (layer F.Cu) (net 3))
 (segment (start 112.03 132.5847) (end 112.03 129.75) (width 0.25) (layer F.Cu) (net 3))
 (segment (start 133.5 122.75) (end 133.5 129.7268) (width 0.25) (layer F.Cu) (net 4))
 (segment (start 112.0056 139.0828) (end 121.3616 129.7268) (width 0.25) (layer B.Cu) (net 4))
 (segment (start 121.3616 129.7268) (end 133.5 129.7268) (width 0.25) (layer B.Cu) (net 4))
 (segment (start 112.0056 139.0828) (end 112.1 139.1772) (width 0.25) (layer F.Cu) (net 4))
 (segment (start 112.1 139.1772) (end 112.1 140) (width 0.25) (layer F.Cu) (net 4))
 (via (at 112.0056 139.0828) (size 0.8) (layers F.Cu B.Cu) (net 4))
 (via (at 133.5 129.7268) (size 0.8) (layers F.Cu B.Cu) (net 4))
 (segment (start 129.5 122.75) (end 129.5 123.8753) (width 0.25) (layer F.Cu) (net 5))
 (segment (start 128.05 126.6) (end 129.1753 126.6) (width 0.25) (layer F.Cu) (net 5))
 (segment (start 129.1753 126.6) (end 129.1753 124.2) (width 0.25) (layer F.Cu) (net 5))
 (segment (start 129.1753 124.2) (end 129.5 123.8753) (width 0.25) (layer F.Cu) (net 5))
 (segment (start 129.5 121.6247) (end 129.5 120.8462) (width 0.25) (layer F.Cu) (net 5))
 (segment (start 129.5 120.8462) (end 128.8964 120.2426) (width 0.25) (layer F.Cu) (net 5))
 (segment (start 129.5 121.6247) (end 130.3 121.6247) (width 0.25) (layer F.Cu) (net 5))
 (segment (start 130.3 122.75) (end 130.3 121.6247) (width 0.25) (layer F.Cu) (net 5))
 (segment (start 129.5 122.75) (end 129.5 121.6247) (width 0.25) (layer F.Cu) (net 5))
 (segment (start 123.4212 118.2921) (end 123.4212 118.9905) (width 0.25) (layer F.Cu) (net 5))
 (segment (start 123.4212 118.9905) (end 122.4117 120) (width 0.25) (layer F.Cu) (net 5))
 (segment (start 122.4117 120) (end 112.79 120) (width 0.25) (layer F.Cu) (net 5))
 (segment (start 122.895 117.995) (end 123.1241 117.995) (width 0.25) (layer F.Cu) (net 5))
 (segment (start 123.1241 117.995) (end 123.4212 118.2921) (width 0.25) (layer F.Cu) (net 5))
 (segment (start 128.8964 120.2426) (end 126.0327 117.3789) (width 0.25) (layer F.Cu) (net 5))
 (segment (start 126.0327 117.3789) (end 124.3344 117.3789) (width 0.25) (layer F.Cu) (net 5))
 (segment (start 124.3344 117.3789) (end 123.4212 118.2921) (width 0.25) (layer F.Cu) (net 5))
 (segment (start 150.3547 124.46) (end 146.1373 120.2426) (width 0.25) (layer B.Cu) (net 5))
 (segment (start 146.1373 120.2426) (end 128.8964 120.2426) (width 0.25) (layer B.Cu) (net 5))
 (segment (start 151.38 124.46) (end 150.3547 124.46) (width 0.25) (layer B.Cu) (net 5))
 (segment (start 112.74 145) (end 130.1488 145) (width 0.25) (layer F.Cu) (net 5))
 (segment (start 130.1488 145) (end 147.7284 127.4204) (width 0.25) (layer F.Cu) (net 5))
 (segment (start 147.7284 127.4204) (end 147.7284 127.0863) (width 0.25) (layer F.Cu) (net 5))
 (segment (start 147.7284 127.0863) (end 150.3547 124.46) (width 0.25) (layer F.Cu) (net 5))
 (segment (start 151.38 124.46) (end 150.3547 124.46) (width 0.25) (layer F.Cu) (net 5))
 (segment (start 112.79 120) (end 112.79 124.95) (width 0.25) (layer F.Cu) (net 5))
 (segment (start 112.79 124.95) (end 112.74 125) (width 0.25) (layer F.Cu) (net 5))
 (via (at 128.8964 120.2426) (size 0.8) (layers F.Cu B.Cu) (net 5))
 (segment (start 118.3781 118.6001) (end 117.1799 118.6001) (width 0.25) (layer F.Cu) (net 6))
 (segment (start 117.1799 118.6001) (end 117.17 118.61) (width 0.25) (layer F.Cu) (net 6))
 (segment (start 148.88 127.66) (end 147.5386 129.0014) (width 0.25) (layer B.Cu) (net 6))
 (segment (start 147.5386 129.0014) (end 128.7794 129.0014) (width 0.25) (layer B.Cu) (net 6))
 (segment (start 128.7794 129.0014) (end 118.3781 118.6001) (width 0.25) (layer B.Cu) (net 6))
 (via (at 118.3781 118.6001) (size 0.8) (layers F.Cu B.Cu) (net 6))
 (segment (start 148.88 124.46) (end 127.3127 124.46) (width 0.25) (layer B.Cu) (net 7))
 (segment (start 127.3127 124.46) (end 120.8227 117.97) (width 0.25) (layer B.Cu) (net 7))
 (segment (start 120.02 117.97) (end 120.8227 117.97) (width 0.25) (layer F.Cu) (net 7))
 (via (at 120.8227 117.97) (size 0.8) (layers F.Cu B.Cu) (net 7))
 (segment (start 136.55 124.2) (end 136.55 122.6564) (width 0.25) (layer F.Cu) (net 8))
 (segment (start 136.55 122.6564) (end 129.8606 115.967) (width 0.25) (layer F.Cu) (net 8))
 (segment (start 129.8606 115.967) (end 118.2831 115.967) (width 0.25) (layer F.Cu) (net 8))
 (segment (start 118.2831 115.967) (end 116.5955 117.6546) (width 0.25) (layer F.Cu) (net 8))
 (segment (start 116.5955 117.6546) (end 116.5955 118.87) (width 0.25) (layer F.Cu) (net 8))
 (segment (start 116.5955 118.87) (end 117.0555 119.33) (width 0.25) (layer F.Cu) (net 8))
 (segment (start 117.0555 119.33) (end 122.2 119.33) (width 0.25) (layer F.Cu) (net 8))
 (segment (start 122.2 119.33) (end 122.895 118.635) (width 0.25) (layer F.Cu) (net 8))
 (segment (start 131.1 122.75) (end 131.1 121.3612) (width 0.25) (layer F.Cu) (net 9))
 (segment (start 131.1 121.3612) (end 126.658 116.9192) (width 0.25) (layer F.Cu) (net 9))
 (segment (start 126.658 116.9192) (end 123.1387 116.9192) (width 0.25) (layer F.Cu) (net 9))
 (segment (start 123.1387 116.9192) (end 121.3131 118.7448) (width 0.25) (layer F.Cu) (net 9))
 (segment (start 121.3131 118.7448) (end 120.1548 118.7448) (width 0.25) (layer F.Cu) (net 9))
 (segment (start 120.1548 118.7448) (end 120.02 118.61) (width 0.25) (layer F.Cu) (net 9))
 (segment (start 131.9 121.6247) (end 131.9 121.5243) (width 0.25) (layer F.Cu) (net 10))
 (segment (start 131.9 121.5243) (end 126.7932 116.4175) (width 0.25) (layer F.Cu) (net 10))
 (segment (start 126.7932 116.4175) (end 118.7225 116.4175) (width 0.25) (layer F.Cu) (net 10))
 (segment (start 118.7225 116.4175) (end 117.17 117.97) (width 0.25) (layer F.Cu) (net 10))
 (segment (start 131.9 122.75) (end 131.9 121.6247) (width 0.25) (layer F.Cu) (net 10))
 (segment (start 132.7 131.25) (end 132.7 132.3753) (width 0.25) (layer F.Cu) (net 11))
 (segment (start 132.7 132.3753) (end 129.0695 132.3753) (width 0.25) (layer F.Cu) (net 11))
 (segment (start 129.0695 132.3753) (end 124.92 128.2258) (width 0.25) (layer F.Cu) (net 11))
 (segment (start 124.92 128.2258) (end 124.92 127.82) (width 0.25) (layer F.Cu) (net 11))
 (segment (start 162.46 99.72) (end 161.7114 99.72) (width 0.25) (layer F.Cu) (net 12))
 (segment (start 161.7114 99.72) (end 147.053 114.3784) (width 0.25) (layer F.Cu) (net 12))
 (segment (start 147.053 114.3784) (end 147.053 127.4589) (width 0.25) (layer F.Cu) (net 12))
 (segment (start 147.053 127.4589) (end 141.6862 132.8257) (width 0.25) (layer F.Cu) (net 12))
 (segment (start 141.6862 132.8257) (end 133.9504 132.8257) (width 0.25) (layer F.Cu) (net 12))
 (segment (start 133.9504 132.8257) (end 133.5 132.3753) (width 0.25) (layer F.Cu) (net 12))
 (segment (start 133.5 131.25) (end 133.5 132.3753) (width 0.25) (layer F.Cu) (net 12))
 (segment (start 162.46 76.2) (end 161.7114 76.2) (width 0.25) (layer F.Cu) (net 13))
 (segment (start 161.7114 76.2) (end 146.5453 91.3661) (width 0.25) (layer F.Cu) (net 13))
 (segment (start 146.5453 91.3661) (end 146.5453 127.3221) (width 0.25) (layer F.Cu) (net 13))
 (segment (start 146.5453 127.3221) (end 141.4921 132.3753) (width 0.25) (layer F.Cu) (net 13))
 (segment (start 141.4921 132.3753) (end 134.3 132.3753) (width 0.25) (layer F.Cu) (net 13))
 (segment (start 134.3 131.25) (end 134.3 132.3753) (width 0.25) (layer F.Cu) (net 13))
 (segment (start 135.1 131.25) (end 136.876 131.25) (width 0.25) (layer F.Cu) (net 14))
 (segment (start 136.876 131.25) (end 142.26 125.866) (width 0.25) (layer F.Cu) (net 14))
 (segment (start 142.26 125.866) (end 142.26 99.72) (width 0.25) (layer F.Cu) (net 14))
 (segment (start 137.6753 129.8) (end 138.5827 128.8926) (width 0.25) (layer F.Cu) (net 15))
 (segment (start 138.5827 128.8926) (end 138.5827 110.7166) (width 0.25) (layer F.Cu) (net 15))
 (segment (start 138.5827 110.7166) (end 137.3865 109.5204) (width 0.25) (layer F.Cu) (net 15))
 (segment (start 137.3865 109.5204) (end 137.3865 87.0113) (width 0.25) (layer F.Cu) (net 15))
 (segment (start 137.3865 87.0113) (end 142.24 82.1578) (width 0.25) (layer F.Cu) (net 15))
 (segment (start 142.24 82.1578) (end 142.24 76.2) (width 0.25) (layer F.Cu) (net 15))
 (segment (start 136.55 129.8) (end 137.6753 129.8) (width 0.25) (layer F.Cu) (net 15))
 (segment (start 136.55 129) (end 137.6753 129) (width 0.25) (layer F.Cu) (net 16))
 (segment (start 127.5726 101.7225) (end 124.0625 101.7225) (width 0.25) (layer B.Cu) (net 16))
 (segment (start 124.0625 101.7225) (end 122.06 99.72) (width 0.25) (layer B.Cu) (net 16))
 (segment (start 137.6753 129) (end 138.1324 128.5429) (width 0.25) (layer F.Cu) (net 16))
 (segment (start 138.1324 128.5429) (end 138.1324 112.2823) (width 0.25) (layer F.Cu) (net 16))
 (segment (start 138.1324 112.2823) (end 127.5726 101.7225) (width 0.25) (layer F.Cu) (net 16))
 (via (at 127.5726 101.7225) (size 0.8) (layers F.Cu B.Cu) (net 16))
 (segment (start 122.06 76.2) (end 122.06 97.2356) (width 0.25) (layer F.Cu) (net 17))
 (segment (start 122.06 97.2356) (end 137.6753 112.8509) (width 0.25) (layer F.Cu) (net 17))
 (segment (start 137.6753 112.8509) (end 137.6753 128.2) (width 0.25) (layer F.Cu) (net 17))
 (segment (start 136.55 128.2) (end 137.6753 128.2) (width 0.25) (layer F.Cu) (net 17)))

